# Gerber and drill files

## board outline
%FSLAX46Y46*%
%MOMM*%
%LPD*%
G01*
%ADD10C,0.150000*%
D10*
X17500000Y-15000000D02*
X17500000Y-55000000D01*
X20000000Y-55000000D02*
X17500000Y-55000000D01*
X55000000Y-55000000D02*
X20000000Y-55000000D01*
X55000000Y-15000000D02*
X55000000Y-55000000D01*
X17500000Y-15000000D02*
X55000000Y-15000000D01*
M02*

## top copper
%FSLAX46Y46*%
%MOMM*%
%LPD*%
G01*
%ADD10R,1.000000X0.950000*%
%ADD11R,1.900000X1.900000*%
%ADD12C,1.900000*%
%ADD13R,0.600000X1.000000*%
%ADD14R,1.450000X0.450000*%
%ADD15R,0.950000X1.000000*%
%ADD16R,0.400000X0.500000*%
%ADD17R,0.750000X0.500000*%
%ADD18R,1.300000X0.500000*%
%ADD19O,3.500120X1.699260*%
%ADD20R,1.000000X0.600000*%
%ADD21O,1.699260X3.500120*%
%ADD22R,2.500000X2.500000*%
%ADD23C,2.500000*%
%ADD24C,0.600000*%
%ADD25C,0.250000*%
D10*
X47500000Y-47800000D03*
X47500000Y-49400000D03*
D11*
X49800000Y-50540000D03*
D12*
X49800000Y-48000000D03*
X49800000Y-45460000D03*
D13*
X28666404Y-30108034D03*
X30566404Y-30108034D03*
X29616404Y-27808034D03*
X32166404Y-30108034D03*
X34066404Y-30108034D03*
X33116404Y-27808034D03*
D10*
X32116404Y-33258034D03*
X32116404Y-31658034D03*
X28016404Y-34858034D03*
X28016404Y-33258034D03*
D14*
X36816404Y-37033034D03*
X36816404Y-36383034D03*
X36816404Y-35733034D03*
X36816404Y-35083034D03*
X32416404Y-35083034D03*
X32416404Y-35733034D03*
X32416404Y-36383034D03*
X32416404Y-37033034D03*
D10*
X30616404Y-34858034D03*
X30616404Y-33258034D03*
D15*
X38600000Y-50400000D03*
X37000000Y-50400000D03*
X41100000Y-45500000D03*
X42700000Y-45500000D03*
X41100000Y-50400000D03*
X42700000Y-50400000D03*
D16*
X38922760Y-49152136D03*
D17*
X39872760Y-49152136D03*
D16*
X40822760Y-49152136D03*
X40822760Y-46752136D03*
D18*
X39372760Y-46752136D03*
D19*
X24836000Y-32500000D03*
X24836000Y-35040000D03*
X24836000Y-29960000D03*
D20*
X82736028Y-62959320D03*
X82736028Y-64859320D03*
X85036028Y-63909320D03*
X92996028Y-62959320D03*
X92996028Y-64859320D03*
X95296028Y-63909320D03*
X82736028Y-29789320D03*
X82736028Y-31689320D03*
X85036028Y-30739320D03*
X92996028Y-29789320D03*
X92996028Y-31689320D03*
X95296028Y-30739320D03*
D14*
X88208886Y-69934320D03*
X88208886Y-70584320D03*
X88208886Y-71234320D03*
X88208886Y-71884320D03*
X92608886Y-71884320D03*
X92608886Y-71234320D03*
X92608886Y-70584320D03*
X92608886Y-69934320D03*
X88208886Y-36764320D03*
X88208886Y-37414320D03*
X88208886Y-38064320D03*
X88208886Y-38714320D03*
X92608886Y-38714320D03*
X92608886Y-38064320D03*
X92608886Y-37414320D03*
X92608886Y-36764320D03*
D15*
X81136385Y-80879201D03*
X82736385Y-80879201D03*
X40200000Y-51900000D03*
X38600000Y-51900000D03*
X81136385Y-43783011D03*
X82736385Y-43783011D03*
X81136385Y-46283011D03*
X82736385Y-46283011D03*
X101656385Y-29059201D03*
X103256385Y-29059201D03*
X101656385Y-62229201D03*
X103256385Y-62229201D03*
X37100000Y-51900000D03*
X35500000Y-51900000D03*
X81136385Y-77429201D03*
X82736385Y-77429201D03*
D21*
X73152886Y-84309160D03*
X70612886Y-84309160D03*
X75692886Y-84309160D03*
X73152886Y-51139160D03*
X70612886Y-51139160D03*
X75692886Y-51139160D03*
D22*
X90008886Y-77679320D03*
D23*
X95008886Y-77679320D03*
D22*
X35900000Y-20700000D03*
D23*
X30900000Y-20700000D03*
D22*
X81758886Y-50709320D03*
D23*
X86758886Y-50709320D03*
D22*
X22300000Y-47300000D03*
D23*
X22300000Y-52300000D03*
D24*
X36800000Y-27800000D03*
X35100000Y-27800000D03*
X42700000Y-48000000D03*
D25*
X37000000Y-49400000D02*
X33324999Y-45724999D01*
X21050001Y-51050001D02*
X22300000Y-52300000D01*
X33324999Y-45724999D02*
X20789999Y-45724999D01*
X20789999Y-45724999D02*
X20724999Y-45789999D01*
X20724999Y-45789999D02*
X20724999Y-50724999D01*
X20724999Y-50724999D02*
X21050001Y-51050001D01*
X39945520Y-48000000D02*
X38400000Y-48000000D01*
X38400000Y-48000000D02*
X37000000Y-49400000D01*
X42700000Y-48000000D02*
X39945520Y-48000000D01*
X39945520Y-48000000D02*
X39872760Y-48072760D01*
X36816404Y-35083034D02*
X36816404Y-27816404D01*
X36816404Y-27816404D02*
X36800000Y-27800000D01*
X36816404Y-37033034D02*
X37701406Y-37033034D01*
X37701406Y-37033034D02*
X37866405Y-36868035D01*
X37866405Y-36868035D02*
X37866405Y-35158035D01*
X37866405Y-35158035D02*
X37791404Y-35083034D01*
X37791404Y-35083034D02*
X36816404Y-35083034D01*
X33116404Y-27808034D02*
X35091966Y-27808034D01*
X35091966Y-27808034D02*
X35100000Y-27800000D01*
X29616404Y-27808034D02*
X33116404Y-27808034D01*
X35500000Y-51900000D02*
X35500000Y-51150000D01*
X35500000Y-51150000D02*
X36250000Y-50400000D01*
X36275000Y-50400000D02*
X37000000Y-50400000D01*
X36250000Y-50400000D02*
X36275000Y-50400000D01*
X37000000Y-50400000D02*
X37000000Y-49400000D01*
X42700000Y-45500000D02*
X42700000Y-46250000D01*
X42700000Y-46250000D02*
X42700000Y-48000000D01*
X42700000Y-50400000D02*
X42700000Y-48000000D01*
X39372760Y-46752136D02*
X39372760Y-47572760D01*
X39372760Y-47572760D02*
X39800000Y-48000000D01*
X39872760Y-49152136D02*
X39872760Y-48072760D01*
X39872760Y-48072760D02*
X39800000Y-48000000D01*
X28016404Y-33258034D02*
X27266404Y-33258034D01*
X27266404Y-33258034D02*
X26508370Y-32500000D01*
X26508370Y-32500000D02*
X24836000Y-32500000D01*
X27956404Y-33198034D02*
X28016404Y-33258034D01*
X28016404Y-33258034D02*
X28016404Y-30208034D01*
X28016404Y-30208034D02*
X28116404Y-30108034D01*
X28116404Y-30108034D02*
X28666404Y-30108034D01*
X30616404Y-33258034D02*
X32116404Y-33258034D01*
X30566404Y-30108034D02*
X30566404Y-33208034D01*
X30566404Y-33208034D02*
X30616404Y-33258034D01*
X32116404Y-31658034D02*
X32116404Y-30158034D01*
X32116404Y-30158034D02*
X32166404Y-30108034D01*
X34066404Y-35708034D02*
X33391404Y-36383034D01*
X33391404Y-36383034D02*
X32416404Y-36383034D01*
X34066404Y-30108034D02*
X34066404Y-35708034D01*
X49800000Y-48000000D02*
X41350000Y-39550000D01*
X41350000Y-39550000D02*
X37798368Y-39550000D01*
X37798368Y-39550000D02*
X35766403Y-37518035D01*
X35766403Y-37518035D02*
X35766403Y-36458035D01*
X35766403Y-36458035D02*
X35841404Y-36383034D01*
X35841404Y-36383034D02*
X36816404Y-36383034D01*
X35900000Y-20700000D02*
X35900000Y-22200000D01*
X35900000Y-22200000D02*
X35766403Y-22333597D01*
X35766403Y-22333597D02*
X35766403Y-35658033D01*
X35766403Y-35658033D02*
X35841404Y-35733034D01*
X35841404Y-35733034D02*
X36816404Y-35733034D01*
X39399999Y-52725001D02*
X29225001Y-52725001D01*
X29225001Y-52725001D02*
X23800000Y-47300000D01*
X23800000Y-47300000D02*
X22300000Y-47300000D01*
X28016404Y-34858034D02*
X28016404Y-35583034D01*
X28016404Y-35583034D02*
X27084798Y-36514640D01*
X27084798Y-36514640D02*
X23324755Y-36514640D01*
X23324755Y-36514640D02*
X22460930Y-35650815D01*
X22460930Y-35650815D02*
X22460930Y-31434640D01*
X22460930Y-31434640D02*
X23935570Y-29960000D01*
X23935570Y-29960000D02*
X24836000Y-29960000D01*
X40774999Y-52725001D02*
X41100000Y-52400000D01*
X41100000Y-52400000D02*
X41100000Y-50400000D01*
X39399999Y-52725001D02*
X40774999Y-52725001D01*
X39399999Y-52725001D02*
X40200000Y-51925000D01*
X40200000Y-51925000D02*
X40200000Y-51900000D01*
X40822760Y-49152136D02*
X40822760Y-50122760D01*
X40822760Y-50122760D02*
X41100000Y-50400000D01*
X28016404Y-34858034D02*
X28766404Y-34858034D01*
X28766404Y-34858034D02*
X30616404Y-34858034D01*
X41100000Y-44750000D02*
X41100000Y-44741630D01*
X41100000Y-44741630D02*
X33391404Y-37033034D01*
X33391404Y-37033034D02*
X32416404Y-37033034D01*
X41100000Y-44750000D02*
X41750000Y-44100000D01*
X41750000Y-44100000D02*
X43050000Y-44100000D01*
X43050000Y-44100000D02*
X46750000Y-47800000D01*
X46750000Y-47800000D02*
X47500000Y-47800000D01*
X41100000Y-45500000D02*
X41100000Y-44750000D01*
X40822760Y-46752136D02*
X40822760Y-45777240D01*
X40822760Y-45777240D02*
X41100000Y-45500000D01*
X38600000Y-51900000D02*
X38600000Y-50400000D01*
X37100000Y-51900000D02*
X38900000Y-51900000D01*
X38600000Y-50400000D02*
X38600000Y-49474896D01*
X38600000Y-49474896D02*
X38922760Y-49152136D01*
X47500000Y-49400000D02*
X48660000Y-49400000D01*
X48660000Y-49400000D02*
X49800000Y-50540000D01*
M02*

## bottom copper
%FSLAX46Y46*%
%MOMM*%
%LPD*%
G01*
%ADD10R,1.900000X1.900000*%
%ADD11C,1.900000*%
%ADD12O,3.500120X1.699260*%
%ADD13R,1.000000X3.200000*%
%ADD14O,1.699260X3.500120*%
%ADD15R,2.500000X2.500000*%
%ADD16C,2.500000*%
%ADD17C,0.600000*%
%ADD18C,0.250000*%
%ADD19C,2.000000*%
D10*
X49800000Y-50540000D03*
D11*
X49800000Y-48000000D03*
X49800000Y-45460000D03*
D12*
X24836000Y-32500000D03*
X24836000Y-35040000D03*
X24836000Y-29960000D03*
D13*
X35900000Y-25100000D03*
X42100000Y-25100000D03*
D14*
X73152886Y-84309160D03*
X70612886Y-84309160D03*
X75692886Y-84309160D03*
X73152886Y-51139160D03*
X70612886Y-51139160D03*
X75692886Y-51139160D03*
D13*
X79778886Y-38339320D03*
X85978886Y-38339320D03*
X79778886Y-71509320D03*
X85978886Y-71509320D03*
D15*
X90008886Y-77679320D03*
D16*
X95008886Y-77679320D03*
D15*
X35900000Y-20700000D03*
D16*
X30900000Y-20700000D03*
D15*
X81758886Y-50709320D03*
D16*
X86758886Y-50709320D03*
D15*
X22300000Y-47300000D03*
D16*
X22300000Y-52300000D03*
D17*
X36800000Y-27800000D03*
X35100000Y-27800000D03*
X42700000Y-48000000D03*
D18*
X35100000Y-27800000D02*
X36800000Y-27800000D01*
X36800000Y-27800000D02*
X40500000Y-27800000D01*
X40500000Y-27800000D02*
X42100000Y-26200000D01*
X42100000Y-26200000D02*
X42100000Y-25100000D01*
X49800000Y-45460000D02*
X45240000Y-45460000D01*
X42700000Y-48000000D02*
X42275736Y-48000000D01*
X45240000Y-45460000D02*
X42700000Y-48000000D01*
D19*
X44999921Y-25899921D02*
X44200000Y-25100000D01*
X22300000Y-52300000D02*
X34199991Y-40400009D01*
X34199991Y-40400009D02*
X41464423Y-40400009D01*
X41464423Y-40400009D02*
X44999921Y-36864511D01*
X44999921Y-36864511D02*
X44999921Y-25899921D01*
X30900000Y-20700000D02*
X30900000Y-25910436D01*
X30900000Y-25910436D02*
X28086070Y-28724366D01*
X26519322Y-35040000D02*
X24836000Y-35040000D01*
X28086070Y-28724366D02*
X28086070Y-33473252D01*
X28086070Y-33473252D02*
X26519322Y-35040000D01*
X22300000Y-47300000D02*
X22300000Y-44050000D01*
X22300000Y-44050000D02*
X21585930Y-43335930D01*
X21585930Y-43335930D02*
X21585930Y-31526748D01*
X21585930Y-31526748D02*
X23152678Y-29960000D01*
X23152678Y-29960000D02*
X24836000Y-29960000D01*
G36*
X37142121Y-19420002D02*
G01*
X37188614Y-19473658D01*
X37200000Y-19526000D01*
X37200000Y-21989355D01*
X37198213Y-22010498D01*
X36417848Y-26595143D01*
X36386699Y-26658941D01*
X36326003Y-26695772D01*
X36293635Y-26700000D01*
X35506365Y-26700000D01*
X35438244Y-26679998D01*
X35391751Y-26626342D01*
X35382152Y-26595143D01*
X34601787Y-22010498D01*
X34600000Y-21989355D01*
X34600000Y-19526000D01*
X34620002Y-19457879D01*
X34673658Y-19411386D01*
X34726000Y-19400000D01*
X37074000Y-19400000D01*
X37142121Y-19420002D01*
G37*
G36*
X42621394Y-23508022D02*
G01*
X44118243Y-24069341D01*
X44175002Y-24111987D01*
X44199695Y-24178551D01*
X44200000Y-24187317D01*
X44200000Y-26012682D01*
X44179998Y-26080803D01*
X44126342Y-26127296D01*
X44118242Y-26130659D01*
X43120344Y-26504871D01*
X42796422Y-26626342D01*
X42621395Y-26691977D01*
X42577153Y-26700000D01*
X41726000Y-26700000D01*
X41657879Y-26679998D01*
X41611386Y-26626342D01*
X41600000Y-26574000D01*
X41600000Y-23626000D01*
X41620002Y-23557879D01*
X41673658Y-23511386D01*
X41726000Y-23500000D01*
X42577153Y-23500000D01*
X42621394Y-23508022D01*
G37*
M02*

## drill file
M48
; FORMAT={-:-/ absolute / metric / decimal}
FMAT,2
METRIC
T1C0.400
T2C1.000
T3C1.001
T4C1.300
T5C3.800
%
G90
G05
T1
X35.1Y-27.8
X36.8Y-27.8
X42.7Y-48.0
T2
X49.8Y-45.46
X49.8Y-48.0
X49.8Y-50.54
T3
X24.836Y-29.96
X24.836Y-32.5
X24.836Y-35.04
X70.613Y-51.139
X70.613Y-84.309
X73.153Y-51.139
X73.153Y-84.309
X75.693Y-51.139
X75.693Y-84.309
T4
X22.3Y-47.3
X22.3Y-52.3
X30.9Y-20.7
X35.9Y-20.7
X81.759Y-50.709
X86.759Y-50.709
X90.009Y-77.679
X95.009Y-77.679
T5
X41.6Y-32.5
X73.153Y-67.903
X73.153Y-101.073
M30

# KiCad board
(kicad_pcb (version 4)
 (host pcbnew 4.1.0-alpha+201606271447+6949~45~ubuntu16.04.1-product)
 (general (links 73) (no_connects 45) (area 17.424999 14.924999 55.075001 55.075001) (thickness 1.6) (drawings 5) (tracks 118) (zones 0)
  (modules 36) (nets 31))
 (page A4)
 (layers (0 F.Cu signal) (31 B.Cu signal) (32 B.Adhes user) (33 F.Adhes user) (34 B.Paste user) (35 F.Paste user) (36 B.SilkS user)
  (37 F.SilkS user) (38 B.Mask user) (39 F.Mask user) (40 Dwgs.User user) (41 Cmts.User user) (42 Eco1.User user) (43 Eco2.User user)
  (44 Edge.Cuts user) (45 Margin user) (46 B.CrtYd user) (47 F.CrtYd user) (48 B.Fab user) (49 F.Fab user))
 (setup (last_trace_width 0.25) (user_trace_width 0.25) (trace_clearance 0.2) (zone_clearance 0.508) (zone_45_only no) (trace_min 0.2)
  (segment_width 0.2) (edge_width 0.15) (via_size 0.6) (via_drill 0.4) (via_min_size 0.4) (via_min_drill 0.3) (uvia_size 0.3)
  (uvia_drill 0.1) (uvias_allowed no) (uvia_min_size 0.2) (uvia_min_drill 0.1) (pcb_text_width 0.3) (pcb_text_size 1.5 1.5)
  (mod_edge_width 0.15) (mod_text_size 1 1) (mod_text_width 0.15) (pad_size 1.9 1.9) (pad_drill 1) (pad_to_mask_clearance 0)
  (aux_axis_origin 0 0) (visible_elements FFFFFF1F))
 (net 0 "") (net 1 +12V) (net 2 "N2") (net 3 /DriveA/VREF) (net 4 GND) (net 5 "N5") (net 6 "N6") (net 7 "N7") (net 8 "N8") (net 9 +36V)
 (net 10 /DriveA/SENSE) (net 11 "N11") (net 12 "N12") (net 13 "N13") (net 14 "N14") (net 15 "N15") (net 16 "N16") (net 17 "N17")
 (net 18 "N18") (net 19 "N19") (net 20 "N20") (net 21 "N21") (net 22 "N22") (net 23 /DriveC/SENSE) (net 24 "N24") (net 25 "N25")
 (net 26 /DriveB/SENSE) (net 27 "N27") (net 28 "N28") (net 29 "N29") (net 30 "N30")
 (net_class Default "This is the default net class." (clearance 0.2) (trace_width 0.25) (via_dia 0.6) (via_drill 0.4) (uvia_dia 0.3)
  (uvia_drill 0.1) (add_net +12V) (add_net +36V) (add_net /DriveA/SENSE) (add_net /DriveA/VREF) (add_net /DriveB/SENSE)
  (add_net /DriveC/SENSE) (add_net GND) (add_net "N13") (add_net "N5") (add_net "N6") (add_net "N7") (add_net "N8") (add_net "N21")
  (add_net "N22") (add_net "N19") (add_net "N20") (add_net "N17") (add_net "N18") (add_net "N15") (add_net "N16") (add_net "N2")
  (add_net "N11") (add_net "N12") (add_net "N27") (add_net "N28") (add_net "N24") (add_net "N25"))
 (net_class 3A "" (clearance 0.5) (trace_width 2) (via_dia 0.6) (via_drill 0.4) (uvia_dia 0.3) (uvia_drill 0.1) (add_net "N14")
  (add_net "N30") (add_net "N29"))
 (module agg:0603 (layer F.Cu) (at 47.5 48.6 270)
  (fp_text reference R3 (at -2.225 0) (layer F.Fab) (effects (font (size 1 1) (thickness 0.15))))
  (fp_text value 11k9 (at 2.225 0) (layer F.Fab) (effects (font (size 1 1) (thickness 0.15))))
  (pad 1 smd rect (at -0.8 0 270) (size 0.95 1) (layers F.Cu F.Paste F.Mask) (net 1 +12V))
  (pad 2 smd rect (at 0.8 0 270) (size 0.95 1) (layers F.Cu F.Paste F.Mask) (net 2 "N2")))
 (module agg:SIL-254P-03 (layer F.Cu) (at 49.8 48 90)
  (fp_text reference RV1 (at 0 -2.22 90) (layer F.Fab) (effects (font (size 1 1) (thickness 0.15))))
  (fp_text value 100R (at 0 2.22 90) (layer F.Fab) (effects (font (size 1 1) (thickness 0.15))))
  (pad 1 thru_hole rect (at -2.54 0 90) (size 1.9 1.9) (drill 1) (layers *.Cu *.Mask F.SilkS) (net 2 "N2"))
  (pad 2 thru_hole circle (at 0 0 90) (size 1.9 1.9) (drill 1) (layers *.Cu *.Mask F.SilkS) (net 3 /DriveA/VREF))
  (pad 3 thru_hole circle (at 2.54 0 90) (size 1.9 1.9) (drill 1) (layers *.Cu *.Mask F.SilkS) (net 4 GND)))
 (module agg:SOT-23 (layer F.Cu) (at 29.616404 28.958034 90)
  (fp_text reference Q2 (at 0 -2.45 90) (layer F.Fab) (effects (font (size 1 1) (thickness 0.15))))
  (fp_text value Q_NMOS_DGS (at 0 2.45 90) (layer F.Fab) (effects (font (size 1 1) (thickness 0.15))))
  (pad 1 smd rect (at -1.15 -0.95 90) (size 1 0.6) (layers F.Cu F.Paste F.Mask) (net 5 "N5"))
  (pad 2 smd rect (at -1.15 0.95 90) (size 1 0.6) (layers F.Cu F.Paste F.Mask) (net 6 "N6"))
  (pad 3 smd rect (at 1.15 0 90) (size 1 0.6) (layers F.Cu F.Paste F.Mask) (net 4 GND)))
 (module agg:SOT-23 (layer F.Cu) (at 33.116404 28.958034 90)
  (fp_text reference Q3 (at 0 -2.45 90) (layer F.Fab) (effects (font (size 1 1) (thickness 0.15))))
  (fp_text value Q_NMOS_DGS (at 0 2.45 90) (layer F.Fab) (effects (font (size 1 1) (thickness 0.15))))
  (pad 1 smd rect (at -1.15 -0.95 90) (size 1 0.6) (layers F.Cu F.Paste F.Mask) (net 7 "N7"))
  (pad 2 smd rect (at -1.15 0.95 90) (size 1 0.6) (layers F.Cu F.Paste F.Mask) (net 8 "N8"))
  (pad 3 smd rect (at 1.15 0 90) (size 1 0.6) (layers F.Cu F.Paste F.Mask) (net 4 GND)))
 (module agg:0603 (layer F.Cu) (at 32.116404 32.458034 90)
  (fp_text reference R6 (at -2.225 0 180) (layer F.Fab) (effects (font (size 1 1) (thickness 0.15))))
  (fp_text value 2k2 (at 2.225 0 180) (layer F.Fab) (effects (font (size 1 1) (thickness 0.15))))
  (pad 1 smd rect (at -0.8 0 90) (size 0.95 1) (layers F.Cu F.Paste F.Mask) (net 6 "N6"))
  (pad 2 smd rect (at 0.8 0 90) (size 0.95 1) (layers F.Cu F.Paste F.Mask) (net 7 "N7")))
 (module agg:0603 (layer F.Cu) (at 28.016404 34.058034 90)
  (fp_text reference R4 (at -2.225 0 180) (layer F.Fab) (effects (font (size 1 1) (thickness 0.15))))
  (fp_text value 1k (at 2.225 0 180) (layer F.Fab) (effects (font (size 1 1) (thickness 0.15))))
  (pad 1 smd rect (at -0.8 0 90) (size 0.95 1) (layers F.Cu F.Paste F.Mask) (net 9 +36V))
  (pad 2 smd rect (at 0.8 0 90) (size 0.95 1) (layers F.Cu F.Paste F.Mask) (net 5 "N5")))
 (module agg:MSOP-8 (layer F.Cu) (at 34.616404 36.058034 180)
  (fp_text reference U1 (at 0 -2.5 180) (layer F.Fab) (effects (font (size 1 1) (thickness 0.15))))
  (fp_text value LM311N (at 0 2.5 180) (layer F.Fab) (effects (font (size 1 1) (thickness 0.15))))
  (pad 1 smd rect (at -2.2 -0.975 180) (size 1.45 0.45) (layers F.Cu F.Paste F.Mask) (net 4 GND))
  (pad 2 smd rect (at -2.2 -0.325 180) (size 1.45 0.45) (layers F.Cu F.Paste F.Mask) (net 3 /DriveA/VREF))
  (pad 3 smd rect (at -2.2 0.325 180) (size 1.45 0.45) (layers F.Cu F.Paste F.Mask) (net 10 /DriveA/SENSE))
  (pad 4 smd rect (at -2.2 0.975 180) (size 1.45 0.45) (layers F.Cu F.Paste F.Mask) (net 4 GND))
  (pad 5 smd rect (at 2.2 0.975 180) (size 1.45 0.45) (layers F.Cu F.Paste F.Mask) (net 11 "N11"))
  (pad 6 smd rect (at 2.2 0.325 180) (size 1.45 0.45) (layers F.Cu F.Paste F.Mask) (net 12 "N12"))
  (pad 7 smd rect (at 2.2 -0.325 180) (size 1.45 0.45) (layers F.Cu F.Paste F.Mask) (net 8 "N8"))
  (pad 8 smd rect (at 2.2 -0.975 180) (size 1.45 0.45) (layers F.Cu F.Paste F.Mask) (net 1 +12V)))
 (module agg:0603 (layer F.Cu) (at 30.616404 34.058034 90)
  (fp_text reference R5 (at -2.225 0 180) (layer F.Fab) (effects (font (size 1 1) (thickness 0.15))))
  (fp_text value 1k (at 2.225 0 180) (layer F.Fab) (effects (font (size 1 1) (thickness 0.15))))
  (pad 1 smd rect (at -0.8 0 90) (size 0.95 1) (layers F.Cu F.Paste F.Mask) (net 9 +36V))
  (pad 2 smd rect (at 0.8 0 90) (size 0.95 1) (layers F.Cu F.Paste F.Mask) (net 6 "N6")))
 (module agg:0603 (layer F.Cu) (at 37.8 50.4 180)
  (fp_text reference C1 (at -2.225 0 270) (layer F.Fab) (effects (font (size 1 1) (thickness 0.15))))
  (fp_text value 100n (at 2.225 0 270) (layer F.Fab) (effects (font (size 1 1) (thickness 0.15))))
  (pad 1 smd rect (at -0.8 0 180) (size 0.95 1) (layers F.Cu F.Paste F.Mask) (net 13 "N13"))
  (pad 2 smd rect (at 0.8 0 180) (size 0.95 1) (layers F.Cu F.Paste F.Mask) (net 4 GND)))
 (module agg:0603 (layer F.Cu) (at 41.9 45.5)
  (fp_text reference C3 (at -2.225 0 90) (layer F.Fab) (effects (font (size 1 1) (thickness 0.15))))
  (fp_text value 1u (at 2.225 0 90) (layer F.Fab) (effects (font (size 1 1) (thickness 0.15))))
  (pad 1 smd rect (at -0.8 0) (size 0.95 1) (layers F.Cu F.Paste F.Mask) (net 1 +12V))
  (pad 2 smd rect (at 0.8 0) (size 0.95 1) (layers F.Cu F.Paste F.Mask) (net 4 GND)))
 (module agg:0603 (layer F.Cu) (at 41.9 50.4)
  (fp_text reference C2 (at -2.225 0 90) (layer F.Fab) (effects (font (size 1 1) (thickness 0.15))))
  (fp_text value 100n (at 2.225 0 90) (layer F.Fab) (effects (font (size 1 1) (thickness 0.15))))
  (pad 1 smd rect (at -0.8 0) (size 0.95 1) (layers F.Cu F.Paste F.Mask) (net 9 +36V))
  (pad 2 smd rect (at 0.8 0) (size 0.95 1) (layers F.Cu F.Paste F.Mask) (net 4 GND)))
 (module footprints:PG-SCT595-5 (layer F.Cu) (at 38.92276 49.152136 90)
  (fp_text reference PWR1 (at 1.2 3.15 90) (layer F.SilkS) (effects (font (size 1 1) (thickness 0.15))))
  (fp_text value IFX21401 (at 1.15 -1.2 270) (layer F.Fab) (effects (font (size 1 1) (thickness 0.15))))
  (pad 1 smd rect (at 0 0 90) (size 0.5 0.4) (layers F.Cu F.Paste F.Mask) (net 13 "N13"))
  (pad 2 smd rect (at 0 0.95 90) (size 0.5 0.75) (layers F.Cu F.Paste F.Mask) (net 4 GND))
  (pad 3 smd rect (at 0 1.9 90) (size 0.5 0.4) (layers F.Cu F.Paste F.Mask) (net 9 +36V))
  (pad 4 smd rect (at 2.4 1.9 90) (size 0.5 0.4) (layers F.Cu F.Paste F.Mask) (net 1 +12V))
  (pad 5 smd rect (at 2.4 0.45 90) (size 0.5 1.3) (layers F.Cu F.Paste F.Mask) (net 4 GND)))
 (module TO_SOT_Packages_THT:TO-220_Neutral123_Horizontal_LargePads (layer B.Cu) (at 24.836 32.5 90)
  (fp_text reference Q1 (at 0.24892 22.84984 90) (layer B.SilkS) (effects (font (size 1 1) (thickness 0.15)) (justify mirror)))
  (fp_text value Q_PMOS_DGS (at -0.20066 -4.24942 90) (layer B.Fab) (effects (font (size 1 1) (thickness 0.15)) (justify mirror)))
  (pad 2 thru_hole oval (at 0 0) (size 3.50012 1.69926) (drill 1.00076) (layers *.Cu *.Mask B.SilkS) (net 5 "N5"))
  (pad 1 thru_hole oval (at -2.54 0) (size 3.50012 1.69926) (drill 1.00076) (layers *.Cu *.Mask B.SilkS) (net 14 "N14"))
  (pad 3 thru_hole oval (at 2.54 0) (size 3.50012 1.69926) (drill 1.00076) (layers *.Cu *.Mask B.SilkS) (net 9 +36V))
  (pad "" np_thru_hole circle (at 0 16.764) (size 3.79984 3.79984) (drill 3.79984) (layers *.Cu *.Mask B.SilkS)))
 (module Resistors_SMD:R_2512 (layer B.Cu) (at 39 25.1)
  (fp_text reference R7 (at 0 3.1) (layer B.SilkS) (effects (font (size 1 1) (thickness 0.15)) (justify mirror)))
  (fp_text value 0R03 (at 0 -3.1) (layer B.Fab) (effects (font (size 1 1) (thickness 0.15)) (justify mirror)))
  (pad 1 smd rect (at -3.1 0) (size 1 3.2) (layers B.Cu B.Paste B.Mask) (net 10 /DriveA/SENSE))
  (pad 2 smd rect (at 3.1 0) (size 1 3.2) (layers B.Cu B.Paste B.Mask) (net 4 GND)))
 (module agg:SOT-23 (layer F.Cu) (at 83.886028 63.90932)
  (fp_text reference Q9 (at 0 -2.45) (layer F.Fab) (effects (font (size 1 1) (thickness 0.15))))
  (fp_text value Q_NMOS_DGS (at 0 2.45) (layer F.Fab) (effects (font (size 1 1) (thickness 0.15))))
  (pad 1 smd rect (at -1.15 -0.95) (size 1 0.6) (layers F.Cu F.Paste F.Mask) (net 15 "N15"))
  (pad 2 smd rect (at -1.15 0.95) (size 1 0.6) (layers F.Cu F.Paste F.Mask) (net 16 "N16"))
  (pad 3 smd rect (at 1.15 0) (size 1 0.6) (layers F.Cu F.Paste F.Mask) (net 4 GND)))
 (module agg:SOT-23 (layer F.Cu) (at 94.146028 63.90932)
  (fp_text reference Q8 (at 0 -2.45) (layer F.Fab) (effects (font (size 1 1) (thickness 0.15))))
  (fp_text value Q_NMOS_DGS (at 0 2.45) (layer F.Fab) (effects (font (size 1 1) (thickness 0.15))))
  (pad 1 smd rect (at -1.15 -0.95) (size 1 0.6) (layers F.Cu F.Paste F.Mask) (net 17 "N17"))
  (pad 2 smd rect (at -1.15 0.95) (size 1 0.6) (layers F.Cu F.Paste F.Mask) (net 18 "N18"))
  (pad 3 smd rect (at 1.15 0) (size 1 0.6) (layers F.Cu F.Paste F.Mask) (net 4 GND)))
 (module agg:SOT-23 (layer F.Cu) (at 83.886028 30.73932)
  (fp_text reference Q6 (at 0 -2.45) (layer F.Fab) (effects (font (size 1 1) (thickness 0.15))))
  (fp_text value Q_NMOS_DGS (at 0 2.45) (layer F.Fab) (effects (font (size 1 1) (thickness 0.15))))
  (pad 1 smd rect (at -1.15 -0.95) (size 1 0.6) (layers F.Cu F.Paste F.Mask) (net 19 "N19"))
  (pad 2 smd rect (at -1.15 0.95) (size 1 0.6) (layers F.Cu F.Paste F.Mask) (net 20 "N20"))
  (pad 3 smd rect (at 1.15 0) (size 1 0.6) (layers F.Cu F.Paste F.Mask) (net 4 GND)))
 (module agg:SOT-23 (layer F.Cu) (at 94.146028 30.73932)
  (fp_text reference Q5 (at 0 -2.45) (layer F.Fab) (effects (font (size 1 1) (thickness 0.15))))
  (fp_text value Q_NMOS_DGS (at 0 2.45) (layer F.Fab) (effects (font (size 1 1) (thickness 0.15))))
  (pad 1 smd rect (at -1.15 -0.95) (size 1 0.6) (layers F.Cu F.Paste F.Mask) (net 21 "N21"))
  (pad 2 smd rect (at -1.15 0.95) (size 1 0.6) (layers F.Cu F.Paste F.Mask) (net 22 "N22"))
  (pad 3 smd rect (at 1.15 0) (size 1 0.6) (layers F.Cu F.Paste F.Mask) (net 4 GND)))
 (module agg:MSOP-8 (layer F.Cu) (at 90.408886 70.90932)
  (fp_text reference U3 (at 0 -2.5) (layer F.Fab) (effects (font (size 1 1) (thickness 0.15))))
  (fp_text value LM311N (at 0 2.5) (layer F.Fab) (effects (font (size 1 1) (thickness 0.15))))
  (pad 1 smd rect (at -2.2 -0.975) (size 1.45 0.45) (layers F.Cu F.Paste F.Mask) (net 4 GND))
  (pad 2 smd rect (at -2.2 -0.325) (size 1.45 0.45) (layers F.Cu F.Paste F.Mask) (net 3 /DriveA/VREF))
  (pad 3 smd rect (at -2.2 0.325) (size 1.45 0.45) (layers F.Cu F.Paste F.Mask) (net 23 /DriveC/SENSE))
  (pad 4 smd rect (at -2.2 0.975) (size 1.45 0.45) (layers F.Cu F.Paste F.Mask) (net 4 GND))
  (pad 5 smd rect (at 2.2 0.975) (size 1.45 0.45) (layers F.Cu F.Paste F.Mask) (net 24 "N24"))
  (pad 6 smd rect (at 2.2 0.325) (size 1.45 0.45) (layers F.Cu F.Paste F.Mask) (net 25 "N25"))
  (pad 7 smd rect (at 2.2 -0.325) (size 1.45 0.45) (layers F.Cu F.Paste F.Mask) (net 16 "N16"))
  (pad 8 smd rect (at 2.2 -0.975) (size 1.45 0.45) (layers F.Cu F.Paste F.Mask) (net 1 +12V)))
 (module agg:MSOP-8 (layer F.Cu) (at 90.408886 37.73932)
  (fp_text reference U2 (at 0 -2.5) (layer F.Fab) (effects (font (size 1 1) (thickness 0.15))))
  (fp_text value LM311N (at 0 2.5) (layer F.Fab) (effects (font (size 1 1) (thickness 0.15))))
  (pad 1 smd rect (at -2.2 -0.975) (size 1.45 0.45) (layers F.Cu F.Paste F.Mask) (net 4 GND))
  (pad 2 smd rect (at -2.2 -0.325) (size 1.45 0.45) (layers F.Cu F.Paste F.Mask) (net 3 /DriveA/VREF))
  (pad 3 smd rect (at -2.2 0.325) (size 1.45 0.45) (layers F.Cu F.Paste F.Mask) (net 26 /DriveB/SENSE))
  (pad 4 smd rect (at -2.2 0.975) (size 1.45 0.45) (layers F.Cu F.Paste F.Mask) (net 4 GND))
  (pad 5 smd rect (at 2.2 0.975) (size 1.45 0.45) (layers F.Cu F.Paste F.Mask) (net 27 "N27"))
  (pad 6 smd rect (at 2.2 0.325) (size 1.45 0.45) (layers F.Cu F.Paste F.Mask) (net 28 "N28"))
  (pad 7 smd rect (at 2.2 -0.325) (size 1.45 0.45) (layers F.Cu F.Paste F.Mask) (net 20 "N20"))
  (pad 8 smd rect (at 2.2 -0.975) (size 1.45 0.45) (layers F.Cu F.Paste F.Mask) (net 1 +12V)))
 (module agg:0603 (layer F.Cu) (at 81.936385 80.879201)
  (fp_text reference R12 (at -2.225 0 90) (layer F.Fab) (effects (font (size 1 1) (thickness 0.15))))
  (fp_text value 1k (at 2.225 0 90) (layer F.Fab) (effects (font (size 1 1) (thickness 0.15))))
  (pad 1 smd rect (at -0.8 0) (size 0.95 1) (layers F.Cu F.Paste F.Mask) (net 9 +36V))
  (pad 2 smd rect (at 0.8 0) (size 0.95 1) (layers F.Cu F.Paste F.Mask) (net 17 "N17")))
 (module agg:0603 (layer F.Cu) (at 39.4 51.9 180)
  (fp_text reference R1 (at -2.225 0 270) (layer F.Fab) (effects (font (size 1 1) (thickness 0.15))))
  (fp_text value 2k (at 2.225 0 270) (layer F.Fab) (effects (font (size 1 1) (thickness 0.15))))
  (pad 1 smd rect (at -0.8 0 180) (size 0.95 1) (layers F.Cu F.Paste F.Mask) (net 9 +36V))
  (pad 2 smd rect (at 0.8 0 180) (size 0.95 1) (layers F.Cu F.Paste F.Mask) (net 13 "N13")))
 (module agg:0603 (layer F.Cu) (at 81.936385 43.783011)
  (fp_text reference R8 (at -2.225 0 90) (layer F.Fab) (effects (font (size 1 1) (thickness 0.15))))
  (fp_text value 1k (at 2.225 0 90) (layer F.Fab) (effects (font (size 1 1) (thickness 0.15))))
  (pad 1 smd rect (at -0.8 0) (size 0.95 1) (layers F.Cu F.Paste F.Mask) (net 9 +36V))
  (pad 2 smd rect (at 0.8 0) (size 0.95 1) (layers F.Cu F.Paste F.Mask) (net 21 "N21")))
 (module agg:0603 (layer F.Cu) (at 81.936385 46.283011)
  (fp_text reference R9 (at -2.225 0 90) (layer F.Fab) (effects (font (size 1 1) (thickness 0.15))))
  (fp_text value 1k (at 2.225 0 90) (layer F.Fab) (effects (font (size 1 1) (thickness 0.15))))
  (pad 1 smd rect (at -0.8 0) (size 0.95 1) (layers F.Cu F.Paste F.Mask) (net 9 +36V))
  (pad 2 smd rect (at 0.8 0) (size 0.95 1) (layers F.Cu F.Paste F.Mask) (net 22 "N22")))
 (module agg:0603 (layer F.Cu) (at 102.456385 29.059201)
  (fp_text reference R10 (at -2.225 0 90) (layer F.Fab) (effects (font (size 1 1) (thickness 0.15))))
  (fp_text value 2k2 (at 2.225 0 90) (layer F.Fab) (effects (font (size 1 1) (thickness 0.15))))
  (pad 1 smd rect (at -0.8 0) (size 0.95 1) (layers F.Cu F.Paste F.Mask) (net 22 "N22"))
  (pad 2 smd rect (at 0.8 0) (size 0.95 1) (layers F.Cu F.Paste F.Mask) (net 19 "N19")))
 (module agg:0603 (layer F.Cu) (at 102.456385 62.229201)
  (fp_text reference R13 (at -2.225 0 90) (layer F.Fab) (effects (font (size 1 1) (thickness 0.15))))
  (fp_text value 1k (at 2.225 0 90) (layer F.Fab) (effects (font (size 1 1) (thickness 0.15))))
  (pad 1 smd rect (at -0.8 0) (size 0.95 1) (layers F.Cu F.Paste F.Mask) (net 9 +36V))
  (pad 2 smd rect (at 0.8 0) (size 0.95 1) (layers F.Cu F.Paste F.Mask) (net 18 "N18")))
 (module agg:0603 (layer F.Cu) (at 36.3 51.9 180)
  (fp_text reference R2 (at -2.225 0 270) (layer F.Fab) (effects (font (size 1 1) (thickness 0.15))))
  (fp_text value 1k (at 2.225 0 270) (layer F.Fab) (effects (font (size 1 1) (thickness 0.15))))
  (pad 1 smd rect (at -0.8 0 180) (size 0.95 1) (layers F.Cu F.Paste F.Mask) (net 13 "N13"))
  (pad 2 smd rect (at 0.8 0 180) (size 0.95 1) (layers F.Cu F.Paste F.Mask) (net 4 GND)))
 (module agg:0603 (layer F.Cu) (at 81.936385 77.429201)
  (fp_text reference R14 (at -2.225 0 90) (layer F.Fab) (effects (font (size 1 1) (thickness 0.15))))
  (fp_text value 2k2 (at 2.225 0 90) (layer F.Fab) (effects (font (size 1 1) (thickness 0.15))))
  (pad 1 smd rect (at -0.8 0) (size 0.95 1) (layers F.Cu F.Paste F.Mask) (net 18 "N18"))
  (pad 2 smd rect (at 0.8 0) (size 0.95 1) (layers F.Cu F.Paste F.Mask) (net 15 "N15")))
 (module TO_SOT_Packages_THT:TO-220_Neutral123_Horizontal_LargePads (layer B.Cu) (at 73.152886 84.30916)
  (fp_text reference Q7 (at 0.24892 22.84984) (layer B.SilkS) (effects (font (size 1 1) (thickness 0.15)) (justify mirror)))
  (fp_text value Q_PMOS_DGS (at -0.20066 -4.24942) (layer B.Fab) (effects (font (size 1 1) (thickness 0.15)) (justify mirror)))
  (pad 2 thru_hole oval (at 0 0 270) (size 3.50012 1.69926) (drill 1.00076) (layers *.Cu *.Mask B.SilkS) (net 17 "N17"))
  (pad 1 thru_hole oval (at -2.54 0 270) (size 3.50012 1.69926) (drill 1.00076) (layers *.Cu *.Mask B.SilkS) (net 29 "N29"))
  (pad 3 thru_hole oval (at 2.54 0 270) (size 3.50012 1.69926) (drill 1.00076) (layers *.Cu *.Mask B.SilkS) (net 9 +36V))
  (pad "" np_thru_hole circle (at 0 16.764 270) (size 3.79984 3.79984) (drill 3.79984) (layers *.Cu *.Mask B.SilkS)))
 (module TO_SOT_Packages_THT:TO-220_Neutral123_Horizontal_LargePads (layer B.Cu) (at 73.152886 51.13916)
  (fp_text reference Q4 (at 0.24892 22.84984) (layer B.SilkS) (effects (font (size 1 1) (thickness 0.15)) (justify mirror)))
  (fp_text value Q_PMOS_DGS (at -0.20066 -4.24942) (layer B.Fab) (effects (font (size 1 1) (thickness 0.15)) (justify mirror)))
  (pad 2 thru_hole oval (at 0 0 270) (size 3.50012 1.69926) (drill 1.00076) (layers *.Cu *.Mask B.SilkS) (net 21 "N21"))
  (pad 1 thru_hole oval (at -2.54 0 270) (size 3.50012 1.69926) (drill 1.00076) (layers *.Cu *.Mask B.SilkS) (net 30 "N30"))
  (pad 3 thru_hole oval (at 2.54 0 270) (size 3.50012 1.69926) (drill 1.00076) (layers *.Cu *.Mask B.SilkS) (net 9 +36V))
  (pad "" np_thru_hole circle (at 0 16.764 270) (size 3.79984 3.79984) (drill 3.79984) (layers *.Cu *.Mask B.SilkS)))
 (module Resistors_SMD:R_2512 (layer B.Cu) (at 82.878886 38.33932)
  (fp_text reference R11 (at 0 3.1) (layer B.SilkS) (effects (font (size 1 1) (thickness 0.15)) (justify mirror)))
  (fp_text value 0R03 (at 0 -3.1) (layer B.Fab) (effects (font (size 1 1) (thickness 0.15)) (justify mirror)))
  (pad 1 smd rect (at -3.1 0) (size 1 3.2) (layers B.Cu B.Paste B.Mask) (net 26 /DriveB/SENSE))
  (pad 2 smd rect (at 3.1 0) (size 1 3.2) (layers B.Cu B.Paste B.Mask) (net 4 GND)))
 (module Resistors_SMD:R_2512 (layer B.Cu) (at 82.878886 71.50932)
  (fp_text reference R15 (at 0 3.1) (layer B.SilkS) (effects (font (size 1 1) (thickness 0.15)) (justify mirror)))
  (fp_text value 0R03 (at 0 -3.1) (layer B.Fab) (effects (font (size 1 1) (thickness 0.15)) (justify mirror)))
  (pad 1 smd rect (at -3.1 0) (size 1 3.2) (layers B.Cu B.Paste B.Mask) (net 23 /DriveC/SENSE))
  (pad 2 smd rect (at 3.1 0) (size 1 3.2) (layers B.Cu B.Paste B.Mask) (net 4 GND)))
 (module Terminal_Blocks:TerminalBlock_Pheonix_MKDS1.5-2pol (layer F.Cu) (at 90.008886 77.67932)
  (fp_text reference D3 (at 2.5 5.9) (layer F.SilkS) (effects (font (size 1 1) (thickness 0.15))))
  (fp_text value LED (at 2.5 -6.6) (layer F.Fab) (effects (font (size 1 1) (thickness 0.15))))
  (pad 1 thru_hole rect (at 0 0) (size 2.5 2.5) (drill 1.3) (layers *.Cu *.Mask F.SilkS) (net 23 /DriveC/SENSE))
  (pad 2 thru_hole circle (at 5 0) (size 2.5 2.5) (drill 1.3) (layers *.Cu *.Mask F.SilkS) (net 29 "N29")))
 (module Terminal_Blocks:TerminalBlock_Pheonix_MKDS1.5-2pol (layer F.Cu) (at 35.9 20.7 180)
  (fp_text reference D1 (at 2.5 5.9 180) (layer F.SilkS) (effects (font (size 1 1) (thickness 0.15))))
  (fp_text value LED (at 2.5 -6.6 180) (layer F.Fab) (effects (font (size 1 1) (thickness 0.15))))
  (pad 1 thru_hole rect (at 0 0 180) (size 2.5 2.5) (drill 1.3) (layers *.Cu *.Mask F.SilkS) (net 10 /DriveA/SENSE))
  (pad 2 thru_hole circle (at 5 0 180) (size 2.5 2.5) (drill 1.3) (layers *.Cu *.Mask F.SilkS) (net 14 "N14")))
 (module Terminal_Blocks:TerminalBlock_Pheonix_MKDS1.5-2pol (layer F.Cu) (at 81.758886 50.70932)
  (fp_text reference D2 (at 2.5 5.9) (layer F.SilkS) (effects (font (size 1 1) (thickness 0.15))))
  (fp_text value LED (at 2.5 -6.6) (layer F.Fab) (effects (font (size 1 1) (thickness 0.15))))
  (pad 1 thru_hole rect (at 0 0) (size 2.5 2.5) (drill 1.3) (layers *.Cu *.Mask F.SilkS) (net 26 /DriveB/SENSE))
  (pad 2 thru_hole circle (at 5 0) (size 2.5 2.5) (drill 1.3) (layers *.Cu *.Mask F.SilkS) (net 30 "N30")))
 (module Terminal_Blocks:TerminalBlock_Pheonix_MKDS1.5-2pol (layer F.Cu) (at 22.3 47.3 270)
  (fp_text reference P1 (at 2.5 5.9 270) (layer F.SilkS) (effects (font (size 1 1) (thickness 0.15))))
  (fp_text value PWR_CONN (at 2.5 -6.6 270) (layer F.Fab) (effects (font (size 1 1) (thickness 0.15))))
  (pad 1 thru_hole rect (at 0 0 270) (size 2.5 2.5) (drill 1.3) (layers *.Cu *.Mask F.SilkS) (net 9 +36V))
  (pad 2 thru_hole circle (at 5 0 270) (size 2.5 2.5) (drill 1.3) (layers *.Cu *.Mask F.SilkS) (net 4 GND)))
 (gr_line (start 17.5 15) (end 17.5 55) (layer Edge.Cuts) (width 0.15))
 (gr_line (start 20 55) (end 17.5 55) (layer Edge.Cuts) (width 0.15))
 (gr_line (start 55 55) (end 20 55) (layer Edge.Cuts) (width 0.15))
 (gr_line (start 55 15) (end 55 55) (layer Edge.Cuts) (width 0.15))
 (gr_line (start 17.5 15) (end 55 15) (layer Edge.Cuts) (width 0.15))
 (segment (start 37 49.4) (end 33.324999 45.724999) (width 0.25) (layer F.Cu) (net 4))
 (segment (start 21.050001 51.050001) (end 22.3 52.3) (width 0.25) (layer F.Cu) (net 4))
 (segment (start 33.324999 45.724999) (end 20.789999 45.724999) (width 0.25) (layer F.Cu) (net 4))
 (segment (start 20.789999 45.724999) (end 20.724999 45.789999) (width 0.25) (layer F.Cu) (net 4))
 (segment (start 20.724999 45.789999) (end 20.724999 50.724999) (width 0.25) (layer F.Cu) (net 4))
 (segment (start 20.724999 50.724999) (end 21.050001 51.050001) (width 0.25) (layer F.Cu) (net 4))
 (segment (start 39.94552 48) (end 38.4 48) (width 0.25) (layer F.Cu) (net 4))
 (segment (start 38.4 48) (end 37 49.4) (width 0.25) (layer F.Cu) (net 4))
 (segment (start 42.7 48) (end 39.94552 48) (width 0.25) (layer F.Cu) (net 4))
 (segment (start 39.94552 48) (end 39.87276 48.07276) (width 0.25) (layer F.Cu) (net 4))
 (segment (start 35.1 27.8) (end 36.8 27.8) (width 0.25) (layer B.Cu) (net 4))
 (segment (start 36.8 27.8) (end 40.5 27.8) (width 0.25) (layer B.Cu) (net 4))
 (segment (start 36.816404 35.083034) (end 36.816404 27.816404) (width 0.25) (layer F.Cu) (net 4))
 (segment (start 36.816404 27.816404) (end 36.8 27.8) (width 0.25) (layer F.Cu) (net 4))
 (via (at 36.8 27.8) (size 0.6) (drill 0.4) (layers F.Cu B.Cu) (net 4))
 (segment (start 36.816404 37.033034) (end 37.701406 37.033034) (width 0.25) (layer F.Cu) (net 4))
 (segment (start 37.701406 37.033034) (end 37.866405 36.868035) (width 0.25) (layer F.Cu) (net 4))
 (segment (start 37.866405 36.868035) (end 37.866405 35.158035) (width 0.25) (layer F.Cu) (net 4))
 (segment (start 37.866405 35.158035) (end 37.791404 35.083034) (width 0.25) (layer F.Cu) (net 4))
 (segment (start 37.791404 35.083034) (end 36.816404 35.083034) (width 0.25) (layer F.Cu) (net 4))
 (segment (start 40.5 27.8) (end 42.1 26.2) (width 0.25) (layer B.Cu) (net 4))
 (segment (start 42.1 26.2) (end 42.1 25.1) (width 0.25) (layer B.Cu) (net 4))
 (segment (start 33.116404 27.808034) (end 35.091966 27.808034) (width 0.25) (layer F.Cu) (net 4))
 (segment (start 35.091966 27.808034) (end 35.1 27.8) (width 0.25) (layer F.Cu) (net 4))
 (via (at 35.1 27.8) (size 0.6) (drill 0.4) (layers F.Cu B.Cu) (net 4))
 (segment (start 29.616404 27.808034) (end 33.116404 27.808034) (width 0.25) (layer F.Cu) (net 4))
 (segment (start 35.5 51.9) (end 35.5 51.15) (width 0.25) (layer F.Cu) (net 4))
 (segment (start 35.5 51.15) (end 36.25 50.4) (width 0.25) (layer F.Cu) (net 4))
 (segment (start 36.275 50.4) (end 37 50.4) (width 0.25) (layer F.Cu) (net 4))
 (segment (start 36.25 50.4) (end 36.275 50.4) (width 0.25) (layer F.Cu) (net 4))
 (segment (start 49.8 45.46) (end 45.24 45.46) (width 0.25) (layer B.Cu) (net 4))
 (segment (start 37 50.4) (end 37 49.4) (width 0.25) (layer F.Cu) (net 4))
 (segment (start 42.7 45.5) (end 42.7 46.25) (width 0.25) (layer F.Cu) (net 4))
 (segment (start 42.7 46.25) (end 42.7 48) (width 0.25) (layer F.Cu) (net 4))
 (segment (start 42.7 50.4) (end 42.7 48) (width 0.25) (layer F.Cu) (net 4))
 (segment (start 39.37276 46.752136) (end 39.37276 47.57276) (width 0.25) (layer F.Cu) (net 4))
 (segment (start 39.37276 47.57276) (end 39.8 48) (width 0.25) (layer F.Cu) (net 4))
 (segment (start 39.87276 49.152136) (end 39.87276 48.07276) (width 0.25) (layer F.Cu) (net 4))
 (segment (start 39.87276 48.07276) (end 39.8 48) (width 0.25) (layer F.Cu) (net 4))
 (segment (start 42.7 48) (end 42.275736 48) (width 0.25) (layer B.Cu) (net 4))
 (segment (start 45.24 45.46) (end 42.7 48) (width 0.25) (layer B.Cu) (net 4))
 (via (at 42.7 48) (size 0.6) (drill 0.4) (layers F.Cu B.Cu) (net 4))
 (segment (start 44.999921 25.899921) (end 44.2 25.1) (width 2) (layer B.Cu) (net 4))
 (segment (start 22.3 52.3) (end 34.199991 40.400009) (width 2) (layer B.Cu) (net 4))
 (segment (start 34.199991 40.400009) (end 41.464423 40.400009) (width 2) (layer B.Cu) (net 4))
 (segment (start 41.464423 40.400009) (end 44.999921 36.864511) (width 2) (layer B.Cu) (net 4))
 (segment (start 44.999921 36.864511) (end 44.999921 25.899921) (width 2) (layer B.Cu) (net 4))
 (segment (start 28.016404 33.258034) (end 27.266404 33.258034) (width 0.25) (layer F.Cu) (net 5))
 (segment (start 27.266404 33.258034) (end 26.50837 32.5) (width 0.25) (layer F.Cu) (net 5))
 (segment (start 26.50837 32.5) (end 24.836 32.5) (width 0.25) (layer F.Cu) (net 5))
 (segment (start 27.956404 33.198034) (end 28.016404 33.258034) (width 0.25) (layer F.Cu) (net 5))
 (segment (start 28.016404 33.258034) (end 28.016404 30.208034) (width 0.25) (layer F.Cu) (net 5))
 (segment (start 28.016404 30.208034) (end 28.116404 30.108034) (width 0.25) (layer F.Cu) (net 5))
 (segment (start 28.116404 30.108034) (end 28.666404 30.108034) (width 0.25) (layer F.Cu) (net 5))
 (segment (start 30.616404 33.258034) (end 32.116404 33.258034) (width 0.25) (layer F.Cu) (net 6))
 (segment (start 30.566404 30.108034) (end 30.566404 33.208034) (width 0.25) (layer F.Cu) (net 6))
 (segment (start 30.566404 33.208034) (end 30.616404 33.258034) (width 0.25) (layer F.Cu) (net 6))
 (segment (start 32.116404 31.658034) (end 32.116404 30.158034) (width 0.25) (layer F.Cu) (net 7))
 (segment (start 32.116404 30.158034) (end 32.166404 30.108034) (width 0.25) (layer F.Cu) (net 7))
 (segment (start 34.066404 35.708034) (end 33.391404 36.383034) (width 0.25) (layer F.Cu) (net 8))
 (segment (start 33.391404 36.383034) (end 32.416404 36.383034) (width 0.25) (layer F.Cu) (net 8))
 (segment (start 34.066404 30.108034) (end 34.066404 35.708034) (width 0.25) (layer F.Cu) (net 8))
 (segment (start 49.8 48) (end 41.35 39.55) (width 0.25) (layer F.Cu) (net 3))
 (segment (start 41.35 39.55) (end 37.798368 39.55) (width 0.25) (layer F.Cu) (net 3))
 (segment (start 37.798368 39.55) (end 35.766403 37.518035) (width 0.25) (layer F.Cu) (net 3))
 (segment (start 35.766403 37.518035) (end 35.766403 36.458035) (width 0.25) (layer F.Cu) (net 3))
 (segment (start 35.766403 36.458035) (end 35.841404 36.383034) (width 0.25) (layer F.Cu) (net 3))
 (segment (start 35.841404 36.383034) (end 36.816404 36.383034) (width 0.25) (layer F.Cu) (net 3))
 (segment (start 35.9 20.7) (end 35.9 22.2) (width 0.25) (layer F.Cu) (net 10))
 (segment (start 35.9 22.2) (end 35.766403 22.333597) (width 0.25) (layer F.Cu) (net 10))
 (segment (start 35.766403 22.333597) (end 35.766403 35.658033) (width 0.25) (layer F.Cu) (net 10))
 (segment (start 35.766403 35.658033) (end 35.841404 35.733034) (width 0.25) (layer F.Cu) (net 10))
 (segment (start 35.841404 35.733034) (end 36.816404 35.733034) (width 0.25) (layer F.Cu) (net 10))
 (segment (start 30.9 20.7) (end 30.9 25.910436) (width 2) (layer B.Cu) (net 14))
 (segment (start 30.9 25.910436) (end 28.08607 28.724366) (width 2) (layer B.Cu) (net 14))
 (segment (start 26.519322 35.04) (end 24.836 35.04) (width 2) (layer B.Cu) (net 14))
 (segment (start 28.08607 28.724366) (end 28.08607 33.473252) (width 2) (layer B.Cu) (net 14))
 (segment (start 28.08607 33.473252) (end 26.519322 35.04) (width 2) (layer B.Cu) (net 14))
 (segment (start 39.399999 52.725001) (end 29.225001 52.725001) (width 0.25) (layer F.Cu) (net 9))
 (segment (start 29.225001 52.725001) (end 23.8 47.3) (width 0.25) (layer F.Cu) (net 9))
 (segment (start 23.8 47.3) (end 22.3 47.3) (width 0.25) (layer F.Cu) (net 9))
 (segment (start 28.016404 34.858034) (end 28.016404 35.583034) (width 0.25) (layer F.Cu) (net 9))
 (segment (start 28.016404 35.583034) (end 27.084798 36.51464) (width 0.25) (layer F.Cu) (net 9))
 (segment (start 27.084798 36.51464) (end 23.324755 36.51464) (width 0.25) (layer F.Cu) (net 9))
 (segment (start 23.324755 36.51464) (end 22.46093 35.650815) (width 0.25) (layer F.Cu) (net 9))
 (segment (start 22.46093 35.650815) (end 22.46093 31.43464) (width 0.25) (layer F.Cu) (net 9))
 (segment (start 22.46093 31.43464) (end 23.93557 29.96) (width 0.25) (layer F.Cu) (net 9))
 (segment (start 23.93557 29.96) (end 24.836 29.96) (width 0.25) (layer F.Cu) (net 9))
 (segment (start 40.774999 52.725001) (end 41.1 52.4) (width 0.25) (layer F.Cu) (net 9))
 (segment (start 41.1 52.4) (end 41.1 50.4) (width 0.25) (layer F.Cu) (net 9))
 (segment (start 39.399999 52.725001) (end 40.774999 52.725001) (width 0.25) (layer F.Cu) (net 9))
 (segment (start 39.399999 52.725001) (end 40.2 51.925) (width 0.25) (layer F.Cu) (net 9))
 (segment (start 40.2 51.925) (end 40.2 51.9) (width 0.25) (layer F.Cu) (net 9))
 (segment (start 40.82276 49.152136) (end 40.82276 50.12276) (width 0.25) (layer F.Cu) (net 9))
 (segment (start 40.82276 50.12276) (end 41.1 50.4) (width 0.25) (layer F.Cu) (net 9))
 (segment (start 28.016404 34.858034) (end 28.766404 34.858034) (width 0.25) (layer F.Cu) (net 9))
 (segment (start 28.766404 34.858034) (end 30.616404 34.858034) (width 0.25) (layer F.Cu) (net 9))
 (segment (start 22.3 47.3) (end 22.3 44.05) (width 2) (layer B.Cu) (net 9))
 (segment (start 22.3 44.05) (end 21.58593 43.33593) (width 2) (layer B.Cu) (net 9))
 (segment (start 21.58593 43.33593) (end 21.58593 31.526748) (width 2) (layer B.Cu) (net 9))
 (segment (start 21.58593 31.526748) (end 23.152678 29.96) (width 2) (layer B.Cu) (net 9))
 (segment (start 23.152678 29.96) (end 24.836 29.96) (width 2) (layer B.Cu) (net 9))
 (segment (start 41.1 44.75) (end 41.1 44.74163) (width 0.25) (layer F.Cu) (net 1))
 (segment (start 41.1 44.74163) (end 33.391404 37.033034) (width 0.25) (layer F.Cu) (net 1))
 (segment (start 33.391404 37.033034) (end 32.416404 37.033034) (width 0.25) (layer F.Cu) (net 1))
 (segment (start 41.1 44.75) (end 41.75 44.1) (width 0.25) (layer F.Cu) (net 1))
 (segment (start 41.75 44.1) (end 43.05 44.1) (width 0.25) (layer F.Cu) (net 1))
 (segment (start 43.05 44.1) (end 46.75 47.8) (width 0.25) (layer F.Cu) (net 1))
 (segment (start 46.75 47.8) (end 47.5 47.8) (width 0.25) (layer F.Cu) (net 1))
 (segment (start 41.1 45.5) (end 41.1 44.75) (width 0.25) (layer F.Cu) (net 1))
 (segment (start 40.82276 46.752136) (end 40.82276 45.77724) (width 0.25) (layer F.Cu) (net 1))
 (segment (start 40.82276 45.77724) (end 41.1 45.5) (width 0.25) (layer F.Cu) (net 1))
 (segment (start 38.6 51.9) (end 38.6 50.4) (width 0.25) (layer F.Cu) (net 13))
 (segment (start 37.1 51.9) (end 38.9 51.9) (width 0.25) (layer F.Cu) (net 13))
 (segment (start 38.6 50.4) (end 38.6 49.474896) (width 0.25) (layer F.Cu) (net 13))
 (segment (start 38.6 49.474896) (end 38.92276 49.152136) (width 0.25) (layer F.Cu) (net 13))
 (segment (start 47.5 49.4) (end 48.66 49.4) (width 0.25) (layer F.Cu) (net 2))
 (segment (start 48.66 49.4) (end 49.8 50.54) (width 0.25) (layer F.Cu) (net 2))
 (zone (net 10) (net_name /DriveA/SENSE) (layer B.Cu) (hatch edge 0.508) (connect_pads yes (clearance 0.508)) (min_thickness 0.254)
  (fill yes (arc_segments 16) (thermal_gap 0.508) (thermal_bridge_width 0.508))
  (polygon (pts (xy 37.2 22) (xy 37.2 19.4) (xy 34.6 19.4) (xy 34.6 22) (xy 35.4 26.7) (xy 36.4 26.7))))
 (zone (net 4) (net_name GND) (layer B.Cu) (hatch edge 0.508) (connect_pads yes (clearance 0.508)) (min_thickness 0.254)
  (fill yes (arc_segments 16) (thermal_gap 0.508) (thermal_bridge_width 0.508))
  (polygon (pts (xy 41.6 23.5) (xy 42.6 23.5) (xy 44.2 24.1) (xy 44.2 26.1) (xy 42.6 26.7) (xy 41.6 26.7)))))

